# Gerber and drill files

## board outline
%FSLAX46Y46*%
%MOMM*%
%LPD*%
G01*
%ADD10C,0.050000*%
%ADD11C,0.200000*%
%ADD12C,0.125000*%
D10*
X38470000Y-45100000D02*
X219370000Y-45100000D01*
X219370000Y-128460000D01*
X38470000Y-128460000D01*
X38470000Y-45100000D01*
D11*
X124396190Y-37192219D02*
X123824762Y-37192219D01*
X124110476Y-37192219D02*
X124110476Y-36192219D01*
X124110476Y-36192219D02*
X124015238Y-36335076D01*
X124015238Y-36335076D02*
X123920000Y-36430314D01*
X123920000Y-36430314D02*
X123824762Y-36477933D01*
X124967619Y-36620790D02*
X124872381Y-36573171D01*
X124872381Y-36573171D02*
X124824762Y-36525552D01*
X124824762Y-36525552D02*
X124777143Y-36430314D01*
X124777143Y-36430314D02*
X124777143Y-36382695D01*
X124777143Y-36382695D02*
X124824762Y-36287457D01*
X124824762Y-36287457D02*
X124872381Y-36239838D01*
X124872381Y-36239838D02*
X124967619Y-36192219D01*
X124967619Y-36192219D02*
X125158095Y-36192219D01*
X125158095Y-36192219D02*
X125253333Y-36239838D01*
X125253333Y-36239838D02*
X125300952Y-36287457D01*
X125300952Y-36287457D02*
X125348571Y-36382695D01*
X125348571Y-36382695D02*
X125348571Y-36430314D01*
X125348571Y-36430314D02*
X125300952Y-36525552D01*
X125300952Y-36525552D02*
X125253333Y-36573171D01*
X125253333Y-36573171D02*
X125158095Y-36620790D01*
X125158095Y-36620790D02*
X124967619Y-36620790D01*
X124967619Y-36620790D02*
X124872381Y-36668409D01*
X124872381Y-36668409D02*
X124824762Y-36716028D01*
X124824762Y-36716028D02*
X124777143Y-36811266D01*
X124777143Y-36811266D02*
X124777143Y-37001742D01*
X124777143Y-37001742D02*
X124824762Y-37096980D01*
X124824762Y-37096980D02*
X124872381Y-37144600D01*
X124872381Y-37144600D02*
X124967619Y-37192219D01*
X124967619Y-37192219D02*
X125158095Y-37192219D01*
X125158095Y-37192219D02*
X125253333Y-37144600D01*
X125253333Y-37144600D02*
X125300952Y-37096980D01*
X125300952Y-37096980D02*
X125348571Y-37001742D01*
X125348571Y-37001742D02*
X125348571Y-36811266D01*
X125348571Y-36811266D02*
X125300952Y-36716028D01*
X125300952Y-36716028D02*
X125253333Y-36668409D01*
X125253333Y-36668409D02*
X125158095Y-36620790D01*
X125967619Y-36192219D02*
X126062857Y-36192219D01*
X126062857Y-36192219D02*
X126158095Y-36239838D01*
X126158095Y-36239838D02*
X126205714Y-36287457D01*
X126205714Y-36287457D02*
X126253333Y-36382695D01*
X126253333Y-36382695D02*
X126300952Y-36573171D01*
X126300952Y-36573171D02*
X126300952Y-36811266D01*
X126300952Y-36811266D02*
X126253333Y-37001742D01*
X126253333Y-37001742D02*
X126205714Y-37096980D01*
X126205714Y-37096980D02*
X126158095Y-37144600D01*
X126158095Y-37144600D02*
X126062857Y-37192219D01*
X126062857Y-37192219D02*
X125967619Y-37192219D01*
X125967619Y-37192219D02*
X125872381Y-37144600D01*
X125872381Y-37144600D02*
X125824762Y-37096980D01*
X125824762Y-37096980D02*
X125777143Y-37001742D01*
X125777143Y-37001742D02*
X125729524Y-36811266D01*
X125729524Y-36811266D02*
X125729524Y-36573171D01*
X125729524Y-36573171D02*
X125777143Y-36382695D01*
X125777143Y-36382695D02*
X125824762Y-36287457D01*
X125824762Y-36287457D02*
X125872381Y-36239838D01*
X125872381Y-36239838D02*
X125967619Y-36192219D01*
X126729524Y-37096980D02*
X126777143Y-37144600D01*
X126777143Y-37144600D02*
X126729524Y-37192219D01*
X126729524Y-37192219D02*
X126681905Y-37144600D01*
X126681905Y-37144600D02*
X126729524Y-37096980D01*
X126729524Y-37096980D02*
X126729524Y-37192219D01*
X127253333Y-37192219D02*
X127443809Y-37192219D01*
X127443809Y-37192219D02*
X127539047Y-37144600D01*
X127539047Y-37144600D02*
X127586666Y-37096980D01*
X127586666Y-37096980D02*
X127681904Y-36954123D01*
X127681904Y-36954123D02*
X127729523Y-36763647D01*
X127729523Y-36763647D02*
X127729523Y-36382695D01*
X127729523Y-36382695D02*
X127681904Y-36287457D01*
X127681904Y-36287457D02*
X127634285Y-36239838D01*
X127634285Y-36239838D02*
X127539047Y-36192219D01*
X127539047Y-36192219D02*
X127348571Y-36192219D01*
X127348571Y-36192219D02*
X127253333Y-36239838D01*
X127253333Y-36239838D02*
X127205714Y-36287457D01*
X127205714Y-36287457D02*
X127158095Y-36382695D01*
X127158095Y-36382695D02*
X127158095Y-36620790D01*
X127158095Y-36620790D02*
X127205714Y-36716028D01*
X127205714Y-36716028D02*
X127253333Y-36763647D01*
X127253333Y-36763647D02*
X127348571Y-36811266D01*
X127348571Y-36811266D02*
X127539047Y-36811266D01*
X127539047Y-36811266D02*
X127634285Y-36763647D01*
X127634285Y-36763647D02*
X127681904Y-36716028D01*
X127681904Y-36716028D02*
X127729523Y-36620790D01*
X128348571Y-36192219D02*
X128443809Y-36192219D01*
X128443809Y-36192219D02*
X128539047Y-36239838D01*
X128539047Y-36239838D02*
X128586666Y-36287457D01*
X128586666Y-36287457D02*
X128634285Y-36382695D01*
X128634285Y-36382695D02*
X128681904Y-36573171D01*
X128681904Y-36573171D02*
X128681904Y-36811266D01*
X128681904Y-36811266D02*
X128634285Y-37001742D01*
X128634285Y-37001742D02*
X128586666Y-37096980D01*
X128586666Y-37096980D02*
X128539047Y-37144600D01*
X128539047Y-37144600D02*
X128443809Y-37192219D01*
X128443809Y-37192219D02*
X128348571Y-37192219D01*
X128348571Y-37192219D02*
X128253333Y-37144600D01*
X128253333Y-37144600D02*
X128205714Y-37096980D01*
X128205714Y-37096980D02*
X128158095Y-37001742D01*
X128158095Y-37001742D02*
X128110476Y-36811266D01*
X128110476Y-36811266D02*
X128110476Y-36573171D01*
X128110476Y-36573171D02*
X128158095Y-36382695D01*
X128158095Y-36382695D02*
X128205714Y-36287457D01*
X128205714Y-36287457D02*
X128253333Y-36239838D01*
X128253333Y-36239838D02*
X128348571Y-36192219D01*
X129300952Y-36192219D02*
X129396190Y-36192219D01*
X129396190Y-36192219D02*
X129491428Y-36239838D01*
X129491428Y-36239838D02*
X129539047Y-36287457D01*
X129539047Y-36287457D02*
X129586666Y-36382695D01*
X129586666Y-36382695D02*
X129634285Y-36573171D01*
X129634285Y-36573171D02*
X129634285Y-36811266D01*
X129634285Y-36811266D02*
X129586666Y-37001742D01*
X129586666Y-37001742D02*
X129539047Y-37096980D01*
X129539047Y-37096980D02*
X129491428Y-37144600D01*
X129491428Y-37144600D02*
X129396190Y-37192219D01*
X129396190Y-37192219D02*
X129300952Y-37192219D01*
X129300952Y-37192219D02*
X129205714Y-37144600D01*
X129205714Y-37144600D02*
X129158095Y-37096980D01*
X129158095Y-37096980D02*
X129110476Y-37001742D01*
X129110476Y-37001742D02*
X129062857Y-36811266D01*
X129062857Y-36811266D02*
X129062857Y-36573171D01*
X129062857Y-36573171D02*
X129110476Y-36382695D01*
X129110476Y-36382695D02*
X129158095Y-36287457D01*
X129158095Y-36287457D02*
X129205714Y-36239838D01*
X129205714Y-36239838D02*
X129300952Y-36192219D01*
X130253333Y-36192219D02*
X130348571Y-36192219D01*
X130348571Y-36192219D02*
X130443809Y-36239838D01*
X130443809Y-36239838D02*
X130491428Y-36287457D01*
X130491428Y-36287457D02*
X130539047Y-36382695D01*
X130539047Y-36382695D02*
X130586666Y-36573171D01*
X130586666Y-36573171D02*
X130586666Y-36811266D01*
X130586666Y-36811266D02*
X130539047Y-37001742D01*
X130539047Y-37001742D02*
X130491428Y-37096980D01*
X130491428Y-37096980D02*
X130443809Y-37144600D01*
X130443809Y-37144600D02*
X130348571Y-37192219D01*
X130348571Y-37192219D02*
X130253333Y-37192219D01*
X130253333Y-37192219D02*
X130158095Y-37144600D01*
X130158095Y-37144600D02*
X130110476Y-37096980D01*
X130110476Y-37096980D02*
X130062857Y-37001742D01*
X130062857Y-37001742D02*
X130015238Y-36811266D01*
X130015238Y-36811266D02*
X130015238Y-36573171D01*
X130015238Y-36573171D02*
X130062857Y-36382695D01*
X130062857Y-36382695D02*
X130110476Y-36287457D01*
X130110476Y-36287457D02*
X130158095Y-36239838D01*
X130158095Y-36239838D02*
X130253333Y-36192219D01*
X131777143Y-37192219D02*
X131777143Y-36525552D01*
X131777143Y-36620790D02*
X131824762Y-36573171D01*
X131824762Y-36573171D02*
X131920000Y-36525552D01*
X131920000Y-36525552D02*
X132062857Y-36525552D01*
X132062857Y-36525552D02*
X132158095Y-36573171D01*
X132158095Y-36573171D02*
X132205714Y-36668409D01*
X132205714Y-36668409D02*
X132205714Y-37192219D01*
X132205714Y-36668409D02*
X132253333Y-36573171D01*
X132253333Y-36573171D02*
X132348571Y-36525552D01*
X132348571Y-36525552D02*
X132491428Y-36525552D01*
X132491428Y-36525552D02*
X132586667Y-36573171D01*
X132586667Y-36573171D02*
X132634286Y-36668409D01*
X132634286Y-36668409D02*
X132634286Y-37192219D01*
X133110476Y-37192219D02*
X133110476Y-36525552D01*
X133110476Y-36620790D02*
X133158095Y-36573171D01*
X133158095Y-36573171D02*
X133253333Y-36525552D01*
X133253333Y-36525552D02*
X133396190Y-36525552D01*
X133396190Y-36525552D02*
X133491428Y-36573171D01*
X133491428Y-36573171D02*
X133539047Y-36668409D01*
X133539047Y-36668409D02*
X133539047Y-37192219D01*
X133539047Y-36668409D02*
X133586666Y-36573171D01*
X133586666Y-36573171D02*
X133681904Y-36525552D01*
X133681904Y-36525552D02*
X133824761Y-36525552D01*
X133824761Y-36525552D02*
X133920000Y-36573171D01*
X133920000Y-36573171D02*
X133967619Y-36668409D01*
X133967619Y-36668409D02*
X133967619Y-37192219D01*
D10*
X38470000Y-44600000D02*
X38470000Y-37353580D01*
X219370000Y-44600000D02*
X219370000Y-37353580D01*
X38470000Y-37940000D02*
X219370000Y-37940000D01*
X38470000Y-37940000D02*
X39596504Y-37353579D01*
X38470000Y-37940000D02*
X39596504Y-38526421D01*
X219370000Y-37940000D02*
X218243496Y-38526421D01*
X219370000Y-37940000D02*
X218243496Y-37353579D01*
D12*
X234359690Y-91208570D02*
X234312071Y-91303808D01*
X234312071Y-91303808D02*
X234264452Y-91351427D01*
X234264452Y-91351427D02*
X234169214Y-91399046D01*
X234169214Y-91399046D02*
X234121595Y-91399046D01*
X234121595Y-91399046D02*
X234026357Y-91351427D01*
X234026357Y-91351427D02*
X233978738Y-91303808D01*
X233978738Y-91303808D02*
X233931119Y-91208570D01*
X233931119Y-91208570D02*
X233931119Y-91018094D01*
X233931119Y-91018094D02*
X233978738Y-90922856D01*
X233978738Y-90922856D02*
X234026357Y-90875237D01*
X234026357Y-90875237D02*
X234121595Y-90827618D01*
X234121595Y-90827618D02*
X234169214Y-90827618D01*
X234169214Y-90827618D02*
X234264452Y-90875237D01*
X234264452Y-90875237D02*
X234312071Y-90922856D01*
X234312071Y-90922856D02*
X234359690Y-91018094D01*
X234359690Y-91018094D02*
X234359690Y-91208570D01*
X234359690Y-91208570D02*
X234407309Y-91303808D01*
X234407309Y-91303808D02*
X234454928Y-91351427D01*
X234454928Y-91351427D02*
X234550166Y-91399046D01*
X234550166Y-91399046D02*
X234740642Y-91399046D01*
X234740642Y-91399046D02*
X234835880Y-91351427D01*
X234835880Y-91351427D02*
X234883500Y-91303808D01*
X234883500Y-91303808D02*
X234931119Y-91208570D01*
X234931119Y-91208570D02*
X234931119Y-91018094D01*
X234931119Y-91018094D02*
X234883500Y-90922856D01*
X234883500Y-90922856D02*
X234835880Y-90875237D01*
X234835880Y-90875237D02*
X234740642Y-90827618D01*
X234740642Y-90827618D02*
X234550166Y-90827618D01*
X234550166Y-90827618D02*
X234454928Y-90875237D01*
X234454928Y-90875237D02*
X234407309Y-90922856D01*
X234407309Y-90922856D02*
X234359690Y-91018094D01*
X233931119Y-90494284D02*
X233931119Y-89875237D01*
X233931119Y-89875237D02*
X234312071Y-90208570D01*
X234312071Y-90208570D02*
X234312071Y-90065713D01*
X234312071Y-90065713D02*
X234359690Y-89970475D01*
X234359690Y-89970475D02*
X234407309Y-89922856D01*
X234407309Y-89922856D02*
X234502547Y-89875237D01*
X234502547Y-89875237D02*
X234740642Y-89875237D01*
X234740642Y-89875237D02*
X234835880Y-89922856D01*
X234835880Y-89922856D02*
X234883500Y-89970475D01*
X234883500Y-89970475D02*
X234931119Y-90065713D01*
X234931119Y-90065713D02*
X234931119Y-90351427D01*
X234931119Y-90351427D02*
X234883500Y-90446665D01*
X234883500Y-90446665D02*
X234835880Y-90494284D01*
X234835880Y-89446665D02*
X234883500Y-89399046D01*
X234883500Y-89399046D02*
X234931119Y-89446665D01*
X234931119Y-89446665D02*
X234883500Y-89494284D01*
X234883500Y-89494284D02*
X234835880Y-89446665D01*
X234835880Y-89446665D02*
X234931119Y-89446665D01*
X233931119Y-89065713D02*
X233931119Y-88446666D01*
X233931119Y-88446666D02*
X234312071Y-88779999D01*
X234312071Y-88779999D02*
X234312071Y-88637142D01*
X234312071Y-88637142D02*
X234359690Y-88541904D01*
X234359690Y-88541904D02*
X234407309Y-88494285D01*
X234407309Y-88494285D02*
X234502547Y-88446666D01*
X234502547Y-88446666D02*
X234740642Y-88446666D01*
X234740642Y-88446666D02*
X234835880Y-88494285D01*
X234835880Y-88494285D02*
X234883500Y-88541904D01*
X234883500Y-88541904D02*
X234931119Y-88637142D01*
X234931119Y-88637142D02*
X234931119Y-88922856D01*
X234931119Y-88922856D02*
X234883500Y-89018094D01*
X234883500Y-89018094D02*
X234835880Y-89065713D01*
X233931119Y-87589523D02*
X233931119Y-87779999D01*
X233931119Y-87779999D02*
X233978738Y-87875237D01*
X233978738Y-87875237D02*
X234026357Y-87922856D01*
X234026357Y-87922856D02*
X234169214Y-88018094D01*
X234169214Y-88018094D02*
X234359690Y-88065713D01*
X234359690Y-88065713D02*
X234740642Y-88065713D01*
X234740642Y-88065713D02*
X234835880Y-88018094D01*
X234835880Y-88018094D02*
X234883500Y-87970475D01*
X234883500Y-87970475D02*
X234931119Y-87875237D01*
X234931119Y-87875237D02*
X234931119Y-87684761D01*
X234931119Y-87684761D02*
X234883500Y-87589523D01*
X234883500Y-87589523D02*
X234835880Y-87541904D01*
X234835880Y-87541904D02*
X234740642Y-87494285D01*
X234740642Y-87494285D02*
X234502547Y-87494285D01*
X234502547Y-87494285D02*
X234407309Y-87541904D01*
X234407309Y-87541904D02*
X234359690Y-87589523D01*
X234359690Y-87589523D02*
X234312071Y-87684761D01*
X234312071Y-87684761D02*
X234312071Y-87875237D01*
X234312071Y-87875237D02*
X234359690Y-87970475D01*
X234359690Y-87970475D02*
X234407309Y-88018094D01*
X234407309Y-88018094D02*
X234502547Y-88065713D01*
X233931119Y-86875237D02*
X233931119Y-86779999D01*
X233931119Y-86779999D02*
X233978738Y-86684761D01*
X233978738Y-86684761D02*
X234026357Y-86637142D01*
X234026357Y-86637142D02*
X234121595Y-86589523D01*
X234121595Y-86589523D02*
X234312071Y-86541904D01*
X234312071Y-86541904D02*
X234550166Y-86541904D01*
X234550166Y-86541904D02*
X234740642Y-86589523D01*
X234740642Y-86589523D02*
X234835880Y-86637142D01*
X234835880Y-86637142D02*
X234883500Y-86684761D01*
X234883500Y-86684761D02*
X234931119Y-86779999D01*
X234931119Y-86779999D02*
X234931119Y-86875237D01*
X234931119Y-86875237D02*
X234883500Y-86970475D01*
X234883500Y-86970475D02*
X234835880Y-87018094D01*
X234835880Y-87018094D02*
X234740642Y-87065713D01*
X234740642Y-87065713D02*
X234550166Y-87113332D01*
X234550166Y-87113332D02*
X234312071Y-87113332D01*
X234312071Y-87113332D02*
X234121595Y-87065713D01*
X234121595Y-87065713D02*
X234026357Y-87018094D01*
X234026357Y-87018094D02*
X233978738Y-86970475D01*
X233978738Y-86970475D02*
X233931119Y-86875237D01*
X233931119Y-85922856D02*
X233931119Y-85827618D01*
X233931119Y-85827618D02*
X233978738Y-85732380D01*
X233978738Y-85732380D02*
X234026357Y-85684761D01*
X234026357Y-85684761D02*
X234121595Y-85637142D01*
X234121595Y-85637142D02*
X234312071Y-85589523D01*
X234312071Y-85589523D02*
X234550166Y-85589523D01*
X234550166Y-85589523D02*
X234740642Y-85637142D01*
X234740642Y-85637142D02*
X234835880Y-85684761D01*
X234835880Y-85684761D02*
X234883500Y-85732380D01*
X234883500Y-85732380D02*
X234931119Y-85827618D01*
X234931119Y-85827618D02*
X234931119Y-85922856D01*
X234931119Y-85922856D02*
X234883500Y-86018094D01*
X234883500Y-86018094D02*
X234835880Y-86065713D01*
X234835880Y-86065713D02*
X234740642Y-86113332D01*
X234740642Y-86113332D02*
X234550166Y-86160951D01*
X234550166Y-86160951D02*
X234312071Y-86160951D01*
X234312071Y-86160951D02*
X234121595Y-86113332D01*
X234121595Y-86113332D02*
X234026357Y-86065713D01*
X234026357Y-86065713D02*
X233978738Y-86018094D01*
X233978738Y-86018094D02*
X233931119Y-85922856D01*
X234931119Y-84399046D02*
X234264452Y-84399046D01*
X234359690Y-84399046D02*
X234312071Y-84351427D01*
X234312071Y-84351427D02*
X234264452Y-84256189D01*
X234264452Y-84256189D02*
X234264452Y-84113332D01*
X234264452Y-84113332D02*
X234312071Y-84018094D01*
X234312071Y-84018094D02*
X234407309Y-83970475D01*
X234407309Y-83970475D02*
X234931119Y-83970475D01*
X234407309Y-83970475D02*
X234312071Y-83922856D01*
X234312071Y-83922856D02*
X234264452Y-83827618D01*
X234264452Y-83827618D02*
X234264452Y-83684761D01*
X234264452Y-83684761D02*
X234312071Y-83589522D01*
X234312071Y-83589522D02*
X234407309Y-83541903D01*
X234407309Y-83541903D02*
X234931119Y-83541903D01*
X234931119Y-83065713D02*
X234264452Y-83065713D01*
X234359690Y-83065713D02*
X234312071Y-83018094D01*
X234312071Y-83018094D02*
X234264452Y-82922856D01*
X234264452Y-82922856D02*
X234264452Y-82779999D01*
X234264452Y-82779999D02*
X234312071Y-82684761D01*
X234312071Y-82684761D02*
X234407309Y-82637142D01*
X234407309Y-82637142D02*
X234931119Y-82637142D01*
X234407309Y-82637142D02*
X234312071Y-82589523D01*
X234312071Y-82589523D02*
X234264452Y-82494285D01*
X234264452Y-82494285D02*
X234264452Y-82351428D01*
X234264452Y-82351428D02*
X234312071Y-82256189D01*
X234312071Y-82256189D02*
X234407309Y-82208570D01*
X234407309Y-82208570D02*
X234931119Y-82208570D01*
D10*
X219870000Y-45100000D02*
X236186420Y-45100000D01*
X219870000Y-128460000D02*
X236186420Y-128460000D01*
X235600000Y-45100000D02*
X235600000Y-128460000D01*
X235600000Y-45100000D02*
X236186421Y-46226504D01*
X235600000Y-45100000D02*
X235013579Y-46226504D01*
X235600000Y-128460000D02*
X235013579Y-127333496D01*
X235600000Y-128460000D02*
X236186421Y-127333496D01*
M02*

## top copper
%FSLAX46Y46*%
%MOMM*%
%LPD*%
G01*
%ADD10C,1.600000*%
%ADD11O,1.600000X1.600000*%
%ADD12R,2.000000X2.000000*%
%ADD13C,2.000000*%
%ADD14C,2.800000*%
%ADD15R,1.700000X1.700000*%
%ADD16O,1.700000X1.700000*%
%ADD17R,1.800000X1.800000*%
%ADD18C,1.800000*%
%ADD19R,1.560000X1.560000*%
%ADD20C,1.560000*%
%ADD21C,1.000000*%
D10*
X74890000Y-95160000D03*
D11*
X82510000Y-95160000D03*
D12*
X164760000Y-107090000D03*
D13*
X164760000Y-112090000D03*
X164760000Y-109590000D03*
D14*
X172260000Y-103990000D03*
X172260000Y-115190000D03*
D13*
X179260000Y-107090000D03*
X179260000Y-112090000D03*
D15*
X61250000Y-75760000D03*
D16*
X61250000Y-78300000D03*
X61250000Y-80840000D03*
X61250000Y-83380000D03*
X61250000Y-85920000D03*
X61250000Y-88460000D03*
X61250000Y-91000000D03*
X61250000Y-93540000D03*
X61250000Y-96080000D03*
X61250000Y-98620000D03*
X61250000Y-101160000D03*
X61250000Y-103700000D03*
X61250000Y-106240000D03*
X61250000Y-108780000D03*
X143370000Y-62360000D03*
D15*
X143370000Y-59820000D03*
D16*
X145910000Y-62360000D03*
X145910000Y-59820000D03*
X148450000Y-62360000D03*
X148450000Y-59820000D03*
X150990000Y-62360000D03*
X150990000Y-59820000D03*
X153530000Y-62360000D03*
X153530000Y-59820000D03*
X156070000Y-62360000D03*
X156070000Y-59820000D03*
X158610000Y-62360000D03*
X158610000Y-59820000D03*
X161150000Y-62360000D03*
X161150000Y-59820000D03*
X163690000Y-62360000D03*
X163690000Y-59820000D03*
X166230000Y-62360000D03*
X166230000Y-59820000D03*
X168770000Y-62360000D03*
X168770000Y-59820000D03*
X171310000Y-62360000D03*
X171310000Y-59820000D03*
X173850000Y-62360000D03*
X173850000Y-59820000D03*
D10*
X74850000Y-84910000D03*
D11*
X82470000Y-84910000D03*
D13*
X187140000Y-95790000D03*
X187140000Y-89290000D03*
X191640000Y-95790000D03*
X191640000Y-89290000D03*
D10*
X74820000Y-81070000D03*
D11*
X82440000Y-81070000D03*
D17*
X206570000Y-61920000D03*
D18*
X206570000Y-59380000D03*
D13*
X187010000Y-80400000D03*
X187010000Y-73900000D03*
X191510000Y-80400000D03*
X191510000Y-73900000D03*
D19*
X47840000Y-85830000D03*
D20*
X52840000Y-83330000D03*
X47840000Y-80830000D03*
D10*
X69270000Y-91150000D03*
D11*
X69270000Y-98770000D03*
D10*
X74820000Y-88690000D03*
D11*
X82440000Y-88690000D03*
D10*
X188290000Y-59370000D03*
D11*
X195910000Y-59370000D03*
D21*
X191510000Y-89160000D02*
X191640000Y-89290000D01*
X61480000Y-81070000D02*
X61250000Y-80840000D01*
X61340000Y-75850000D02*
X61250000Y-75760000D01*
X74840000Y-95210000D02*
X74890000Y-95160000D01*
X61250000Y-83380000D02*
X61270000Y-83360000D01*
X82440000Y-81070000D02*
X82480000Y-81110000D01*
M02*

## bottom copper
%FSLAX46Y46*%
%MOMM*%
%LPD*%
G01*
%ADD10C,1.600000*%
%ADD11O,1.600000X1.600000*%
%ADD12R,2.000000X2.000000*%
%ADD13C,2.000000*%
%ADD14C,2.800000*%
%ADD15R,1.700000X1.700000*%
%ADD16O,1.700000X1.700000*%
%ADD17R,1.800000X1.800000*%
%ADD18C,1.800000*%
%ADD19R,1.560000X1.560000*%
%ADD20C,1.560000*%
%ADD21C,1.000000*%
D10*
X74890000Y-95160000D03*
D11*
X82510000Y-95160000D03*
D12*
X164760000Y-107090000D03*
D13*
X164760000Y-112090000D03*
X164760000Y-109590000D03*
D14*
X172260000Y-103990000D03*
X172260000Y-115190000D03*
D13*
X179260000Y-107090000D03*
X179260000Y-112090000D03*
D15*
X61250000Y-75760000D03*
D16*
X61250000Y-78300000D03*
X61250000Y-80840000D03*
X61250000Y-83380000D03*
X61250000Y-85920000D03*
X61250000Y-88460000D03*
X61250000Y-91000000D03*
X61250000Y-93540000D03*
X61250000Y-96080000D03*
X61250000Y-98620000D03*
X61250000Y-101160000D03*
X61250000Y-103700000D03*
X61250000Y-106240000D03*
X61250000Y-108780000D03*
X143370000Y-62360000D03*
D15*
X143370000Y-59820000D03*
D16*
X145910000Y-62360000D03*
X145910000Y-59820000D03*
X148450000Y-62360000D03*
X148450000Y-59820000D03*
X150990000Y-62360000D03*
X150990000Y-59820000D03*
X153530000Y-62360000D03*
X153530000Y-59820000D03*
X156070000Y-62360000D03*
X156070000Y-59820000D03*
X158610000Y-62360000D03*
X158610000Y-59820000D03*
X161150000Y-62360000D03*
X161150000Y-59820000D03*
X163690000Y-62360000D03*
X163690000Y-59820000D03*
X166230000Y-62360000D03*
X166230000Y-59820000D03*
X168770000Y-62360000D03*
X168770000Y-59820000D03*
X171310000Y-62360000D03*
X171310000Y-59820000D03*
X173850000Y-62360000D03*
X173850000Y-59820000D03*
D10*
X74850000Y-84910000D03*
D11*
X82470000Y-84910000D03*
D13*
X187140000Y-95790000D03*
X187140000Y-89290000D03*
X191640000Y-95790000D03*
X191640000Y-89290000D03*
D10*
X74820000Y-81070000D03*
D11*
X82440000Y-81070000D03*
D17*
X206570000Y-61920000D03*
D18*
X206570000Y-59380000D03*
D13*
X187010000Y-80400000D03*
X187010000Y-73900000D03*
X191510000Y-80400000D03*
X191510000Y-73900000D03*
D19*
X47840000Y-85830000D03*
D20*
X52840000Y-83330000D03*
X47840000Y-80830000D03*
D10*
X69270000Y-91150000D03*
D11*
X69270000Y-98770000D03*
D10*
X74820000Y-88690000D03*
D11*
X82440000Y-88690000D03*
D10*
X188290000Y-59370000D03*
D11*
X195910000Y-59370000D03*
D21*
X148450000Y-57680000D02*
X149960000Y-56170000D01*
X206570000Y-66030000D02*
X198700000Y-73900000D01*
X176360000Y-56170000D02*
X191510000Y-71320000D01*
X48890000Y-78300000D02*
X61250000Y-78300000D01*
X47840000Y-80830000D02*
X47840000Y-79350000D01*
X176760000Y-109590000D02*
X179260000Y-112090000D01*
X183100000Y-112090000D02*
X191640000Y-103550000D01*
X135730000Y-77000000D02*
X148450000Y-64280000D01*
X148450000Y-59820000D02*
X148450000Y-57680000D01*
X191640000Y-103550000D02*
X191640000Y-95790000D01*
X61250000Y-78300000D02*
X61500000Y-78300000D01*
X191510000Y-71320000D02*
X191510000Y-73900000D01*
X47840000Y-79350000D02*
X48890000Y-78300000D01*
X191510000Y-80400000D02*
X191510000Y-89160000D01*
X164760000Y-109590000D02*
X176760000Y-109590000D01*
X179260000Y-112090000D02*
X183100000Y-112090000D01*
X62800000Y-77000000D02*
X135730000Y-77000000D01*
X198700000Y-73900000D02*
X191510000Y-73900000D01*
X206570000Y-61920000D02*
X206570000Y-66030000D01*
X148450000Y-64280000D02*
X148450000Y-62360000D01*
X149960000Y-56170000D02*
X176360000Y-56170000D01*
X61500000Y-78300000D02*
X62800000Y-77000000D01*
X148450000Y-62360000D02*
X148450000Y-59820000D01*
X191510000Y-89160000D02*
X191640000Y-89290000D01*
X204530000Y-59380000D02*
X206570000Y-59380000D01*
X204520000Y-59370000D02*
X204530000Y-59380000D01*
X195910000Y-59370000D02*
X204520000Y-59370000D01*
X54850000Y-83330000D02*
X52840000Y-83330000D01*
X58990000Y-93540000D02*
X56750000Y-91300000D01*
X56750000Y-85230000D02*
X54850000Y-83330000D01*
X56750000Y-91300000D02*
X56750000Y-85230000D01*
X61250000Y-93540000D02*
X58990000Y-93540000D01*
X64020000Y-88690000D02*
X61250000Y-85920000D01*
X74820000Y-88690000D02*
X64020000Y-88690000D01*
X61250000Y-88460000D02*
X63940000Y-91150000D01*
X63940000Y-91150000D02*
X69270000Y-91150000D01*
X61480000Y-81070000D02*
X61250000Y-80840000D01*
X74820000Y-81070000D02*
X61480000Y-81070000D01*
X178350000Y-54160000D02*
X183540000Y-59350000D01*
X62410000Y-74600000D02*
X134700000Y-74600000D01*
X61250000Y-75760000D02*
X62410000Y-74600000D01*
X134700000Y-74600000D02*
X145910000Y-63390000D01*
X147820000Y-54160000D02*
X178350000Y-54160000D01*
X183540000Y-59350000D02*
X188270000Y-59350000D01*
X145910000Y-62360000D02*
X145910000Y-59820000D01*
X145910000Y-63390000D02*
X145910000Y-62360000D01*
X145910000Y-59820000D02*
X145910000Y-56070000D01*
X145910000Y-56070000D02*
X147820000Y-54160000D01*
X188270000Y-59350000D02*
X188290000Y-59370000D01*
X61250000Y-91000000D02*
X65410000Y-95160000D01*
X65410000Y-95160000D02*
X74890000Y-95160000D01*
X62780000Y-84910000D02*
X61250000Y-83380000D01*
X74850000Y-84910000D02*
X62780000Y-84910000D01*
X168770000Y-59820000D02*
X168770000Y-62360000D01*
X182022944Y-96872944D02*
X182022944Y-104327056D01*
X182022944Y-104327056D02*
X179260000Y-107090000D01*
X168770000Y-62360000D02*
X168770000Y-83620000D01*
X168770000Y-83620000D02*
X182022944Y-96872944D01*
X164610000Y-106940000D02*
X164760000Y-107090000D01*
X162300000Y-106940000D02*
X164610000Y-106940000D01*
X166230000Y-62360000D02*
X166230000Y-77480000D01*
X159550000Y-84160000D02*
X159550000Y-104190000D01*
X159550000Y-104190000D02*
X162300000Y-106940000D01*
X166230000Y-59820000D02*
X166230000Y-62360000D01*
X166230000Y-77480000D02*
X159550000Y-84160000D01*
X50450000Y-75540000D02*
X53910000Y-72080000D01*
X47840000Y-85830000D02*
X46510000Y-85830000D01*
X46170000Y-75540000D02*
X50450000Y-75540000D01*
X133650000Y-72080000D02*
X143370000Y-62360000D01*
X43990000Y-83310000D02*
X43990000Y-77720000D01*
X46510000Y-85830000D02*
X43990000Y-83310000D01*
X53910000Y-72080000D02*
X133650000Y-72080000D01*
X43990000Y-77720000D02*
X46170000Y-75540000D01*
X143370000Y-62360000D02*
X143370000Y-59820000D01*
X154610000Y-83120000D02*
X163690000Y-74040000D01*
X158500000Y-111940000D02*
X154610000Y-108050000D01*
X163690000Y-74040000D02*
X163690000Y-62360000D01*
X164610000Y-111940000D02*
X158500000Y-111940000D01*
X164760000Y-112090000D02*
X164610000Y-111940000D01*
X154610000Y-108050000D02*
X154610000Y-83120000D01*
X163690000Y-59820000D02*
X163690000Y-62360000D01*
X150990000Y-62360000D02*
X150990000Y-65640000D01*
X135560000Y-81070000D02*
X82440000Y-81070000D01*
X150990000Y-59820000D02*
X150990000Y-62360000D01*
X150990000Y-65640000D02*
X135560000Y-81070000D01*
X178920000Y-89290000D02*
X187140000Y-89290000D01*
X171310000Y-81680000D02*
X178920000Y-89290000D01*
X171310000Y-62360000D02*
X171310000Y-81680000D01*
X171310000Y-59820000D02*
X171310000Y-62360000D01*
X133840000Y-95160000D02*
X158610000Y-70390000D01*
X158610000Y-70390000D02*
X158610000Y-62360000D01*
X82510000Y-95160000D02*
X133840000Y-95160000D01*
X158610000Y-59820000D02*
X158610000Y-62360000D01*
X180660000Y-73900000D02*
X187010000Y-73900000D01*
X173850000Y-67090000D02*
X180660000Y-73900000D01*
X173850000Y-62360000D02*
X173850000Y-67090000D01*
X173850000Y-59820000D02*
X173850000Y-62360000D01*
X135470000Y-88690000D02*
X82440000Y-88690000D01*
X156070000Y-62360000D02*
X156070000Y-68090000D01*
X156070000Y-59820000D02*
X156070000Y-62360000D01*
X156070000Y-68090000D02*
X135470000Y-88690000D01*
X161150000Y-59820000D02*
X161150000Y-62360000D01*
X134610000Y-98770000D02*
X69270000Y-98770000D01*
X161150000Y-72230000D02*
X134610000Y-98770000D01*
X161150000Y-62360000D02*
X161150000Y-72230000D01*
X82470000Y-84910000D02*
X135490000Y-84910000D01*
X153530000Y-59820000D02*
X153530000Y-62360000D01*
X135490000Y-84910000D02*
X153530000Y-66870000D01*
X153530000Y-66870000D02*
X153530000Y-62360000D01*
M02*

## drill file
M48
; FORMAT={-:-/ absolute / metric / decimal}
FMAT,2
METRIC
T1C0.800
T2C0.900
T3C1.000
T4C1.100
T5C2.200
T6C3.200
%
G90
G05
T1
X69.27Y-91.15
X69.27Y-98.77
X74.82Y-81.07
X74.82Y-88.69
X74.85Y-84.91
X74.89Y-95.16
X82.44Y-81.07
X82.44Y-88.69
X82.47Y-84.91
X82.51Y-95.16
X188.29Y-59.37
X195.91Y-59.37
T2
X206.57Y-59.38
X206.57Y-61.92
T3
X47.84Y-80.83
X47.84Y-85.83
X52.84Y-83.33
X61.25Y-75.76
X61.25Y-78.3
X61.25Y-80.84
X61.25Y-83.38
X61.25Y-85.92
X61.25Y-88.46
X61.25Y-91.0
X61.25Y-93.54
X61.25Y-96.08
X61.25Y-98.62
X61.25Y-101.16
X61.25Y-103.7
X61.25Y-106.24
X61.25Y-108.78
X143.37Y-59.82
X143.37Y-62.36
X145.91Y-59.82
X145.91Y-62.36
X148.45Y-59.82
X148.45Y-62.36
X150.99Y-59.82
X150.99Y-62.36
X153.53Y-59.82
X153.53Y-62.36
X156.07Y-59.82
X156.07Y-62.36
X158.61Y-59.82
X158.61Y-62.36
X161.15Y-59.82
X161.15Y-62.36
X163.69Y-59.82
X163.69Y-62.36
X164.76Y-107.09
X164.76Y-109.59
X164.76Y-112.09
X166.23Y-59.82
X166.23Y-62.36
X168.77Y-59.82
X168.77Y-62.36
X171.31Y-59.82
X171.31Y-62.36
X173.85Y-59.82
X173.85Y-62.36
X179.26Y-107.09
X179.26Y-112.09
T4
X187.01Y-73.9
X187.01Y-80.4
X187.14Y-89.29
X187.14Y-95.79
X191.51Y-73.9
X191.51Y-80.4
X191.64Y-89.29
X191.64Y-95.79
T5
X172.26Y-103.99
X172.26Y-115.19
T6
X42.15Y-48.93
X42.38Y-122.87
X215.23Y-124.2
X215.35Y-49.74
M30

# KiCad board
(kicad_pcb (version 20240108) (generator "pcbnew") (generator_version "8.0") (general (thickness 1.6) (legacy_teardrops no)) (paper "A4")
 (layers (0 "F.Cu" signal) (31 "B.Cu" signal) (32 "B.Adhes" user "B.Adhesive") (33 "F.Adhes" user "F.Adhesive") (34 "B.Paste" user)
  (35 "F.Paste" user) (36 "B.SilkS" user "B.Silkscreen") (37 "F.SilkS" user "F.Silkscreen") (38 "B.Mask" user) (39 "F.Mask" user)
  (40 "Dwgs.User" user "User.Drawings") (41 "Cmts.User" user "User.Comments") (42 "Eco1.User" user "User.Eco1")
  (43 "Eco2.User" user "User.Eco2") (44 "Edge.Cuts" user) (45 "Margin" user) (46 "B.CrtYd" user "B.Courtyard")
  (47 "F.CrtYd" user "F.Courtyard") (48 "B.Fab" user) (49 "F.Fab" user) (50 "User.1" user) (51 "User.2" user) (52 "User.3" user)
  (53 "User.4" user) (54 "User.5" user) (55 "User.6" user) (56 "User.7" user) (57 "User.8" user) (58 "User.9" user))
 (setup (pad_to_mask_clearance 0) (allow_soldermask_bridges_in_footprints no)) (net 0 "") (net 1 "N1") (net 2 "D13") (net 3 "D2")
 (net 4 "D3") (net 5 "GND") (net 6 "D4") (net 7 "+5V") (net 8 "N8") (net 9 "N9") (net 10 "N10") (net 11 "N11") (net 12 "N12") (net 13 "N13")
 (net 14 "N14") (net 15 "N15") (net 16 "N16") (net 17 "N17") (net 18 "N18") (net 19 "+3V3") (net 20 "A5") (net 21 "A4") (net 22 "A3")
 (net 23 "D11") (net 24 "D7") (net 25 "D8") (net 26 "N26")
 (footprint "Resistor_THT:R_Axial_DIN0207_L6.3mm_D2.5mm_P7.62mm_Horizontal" (layer "F.Cu") (at 74.89 95.16)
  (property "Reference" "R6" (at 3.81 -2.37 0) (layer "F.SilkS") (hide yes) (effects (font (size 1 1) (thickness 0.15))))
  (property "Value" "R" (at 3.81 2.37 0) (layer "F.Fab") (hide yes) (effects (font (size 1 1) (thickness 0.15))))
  (pad "1" thru_hole circle (at 0 0) (size 1.6 1.6) (drill 0.8) (layers "*.Cu" "*.Mask") (remove_unused_layers no) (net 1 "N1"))
  (pad "2" thru_hole oval (at 7.62 0) (size 1.6 1.6) (drill 0.8) (layers "*.Cu" "*.Mask") (remove_unused_layers no) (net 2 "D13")))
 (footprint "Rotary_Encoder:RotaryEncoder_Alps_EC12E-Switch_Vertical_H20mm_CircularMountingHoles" (layer "F.Cu") (at 164.76 107.09)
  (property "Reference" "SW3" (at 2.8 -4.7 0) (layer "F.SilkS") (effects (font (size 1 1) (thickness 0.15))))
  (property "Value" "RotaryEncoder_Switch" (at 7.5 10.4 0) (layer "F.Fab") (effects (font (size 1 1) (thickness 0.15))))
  (pad "A" thru_hole rect (at 0 0) (size 2 2) (drill 1) (layers "*.Cu" "*.Mask") (remove_unused_layers no) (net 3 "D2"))
  (pad "B" thru_hole circle (at 0 5) (size 2 2) (drill 1) (layers "*.Cu" "*.Mask") (remove_unused_layers no) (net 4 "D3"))
  (pad "C" thru_hole circle (at 0 2.5) (size 2 2) (drill 1) (layers "*.Cu" "*.Mask") (remove_unused_layers no) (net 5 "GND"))
  (pad "MP" thru_hole circle (at 7.5 -3.1) (size 2.8 2.8) (drill 2.2) (layers "*.Cu" "*.Mask") (remove_unused_layers no))
  (pad "MP" thru_hole circle (at 7.5 8.1) (size 2.8 2.8) (drill 2.2) (layers "*.Cu" "*.Mask") (remove_unused_layers no))
  (pad "S1" thru_hole circle (at 14.5 0) (size 2 2) (drill 1) (layers "*.Cu" "*.Mask") (remove_unused_layers no) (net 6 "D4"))
  (pad "S2" thru_hole circle (at 14.5 5) (size 2 2) (drill 1) (layers "*.Cu" "*.Mask") (remove_unused_layers no) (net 5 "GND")))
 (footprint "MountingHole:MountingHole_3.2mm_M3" (layer "F.Cu") (at 215.23 124.2)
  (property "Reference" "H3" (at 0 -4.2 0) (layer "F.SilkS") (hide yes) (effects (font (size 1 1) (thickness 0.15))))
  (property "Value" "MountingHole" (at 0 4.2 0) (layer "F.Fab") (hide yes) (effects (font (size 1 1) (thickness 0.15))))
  (pad "" np_thru_hole circle (at 0 0) (size 3.2 3.2) (drill 3.2) (layers "*.Cu" "*.Mask")))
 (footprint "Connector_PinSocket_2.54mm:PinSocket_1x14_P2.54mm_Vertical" (layer "F.Cu") (at 61.25 75.76)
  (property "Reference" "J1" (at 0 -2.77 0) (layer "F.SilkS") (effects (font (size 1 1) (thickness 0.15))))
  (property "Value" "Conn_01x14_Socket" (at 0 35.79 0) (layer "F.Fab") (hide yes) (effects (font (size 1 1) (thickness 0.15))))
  (pad "1" thru_hole rect (at 0 0) (size 1.7 1.7) (drill 1) (layers "*.Cu" "*.Mask") (remove_unused_layers no) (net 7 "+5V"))
  (pad "2" thru_hole oval (at 0 2.54) (size 1.7 1.7) (drill 1) (layers "*.Cu" "*.Mask") (remove_unused_layers no) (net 5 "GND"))
  (pad "3" thru_hole oval (at 0 5.08) (size 1.7 1.7) (drill 1) (layers "*.Cu" "*.Mask") (remove_unused_layers no) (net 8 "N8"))
  (pad "4" thru_hole oval (at 0 7.62) (size 1.7 1.7) (drill 1) (layers "*.Cu" "*.Mask") (remove_unused_layers no) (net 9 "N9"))
  (pad "5" thru_hole oval (at 0 10.16) (size 1.7 1.7) (drill 1) (layers "*.Cu" "*.Mask") (remove_unused_layers no) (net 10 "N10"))
  (pad "6" thru_hole oval (at 0 12.7) (size 1.7 1.7) (drill 1) (layers "*.Cu" "*.Mask") (remove_unused_layers no) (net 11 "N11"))
  (pad "7" thru_hole oval (at 0 15.24) (size 1.7 1.7) (drill 1) (layers "*.Cu" "*.Mask") (remove_unused_layers no) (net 1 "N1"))
  (pad "8" thru_hole oval (at 0 17.78) (size 1.7 1.7) (drill 1) (layers "*.Cu" "*.Mask") (remove_unused_layers no) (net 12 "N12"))
  (pad "9" thru_hole oval (at 0 20.32) (size 1.7 1.7) (drill 1) (layers "*.Cu" "*.Mask") (remove_unused_layers no) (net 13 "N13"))
  (pad "10" thru_hole oval (at 0 22.86) (size 1.7 1.7) (drill 1) (layers "*.Cu" "*.Mask") (remove_unused_layers no) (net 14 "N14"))
  (pad "11" thru_hole oval (at 0 25.4) (size 1.7 1.7) (drill 1) (layers "*.Cu" "*.Mask") (remove_unused_layers no) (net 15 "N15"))
  (pad "12" thru_hole oval (at 0 27.94) (size 1.7 1.7) (drill 1) (layers "*.Cu" "*.Mask") (remove_unused_layers no) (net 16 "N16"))
  (pad "13" thru_hole oval (at 0 30.48) (size 1.7 1.7) (drill 1) (layers "*.Cu" "*.Mask") (remove_unused_layers no) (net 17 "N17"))
  (pad "14" thru_hole oval (at 0 33.02) (size 1.7 1.7) (drill 1) (layers "*.Cu" "*.Mask") (remove_unused_layers no) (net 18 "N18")))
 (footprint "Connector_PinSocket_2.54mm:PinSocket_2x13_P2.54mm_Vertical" (layer "F.Cu") (at 143.37 59.82 90)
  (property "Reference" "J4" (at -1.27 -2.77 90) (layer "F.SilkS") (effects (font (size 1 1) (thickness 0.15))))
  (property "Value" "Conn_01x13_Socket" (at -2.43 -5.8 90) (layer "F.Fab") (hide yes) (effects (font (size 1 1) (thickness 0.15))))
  (pad "1" thru_hole oval (at -2.54 0 90) (size 1.7 1.7) (drill 1) (layers "*.Cu" "*.Mask") (remove_unused_layers no) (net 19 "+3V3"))
  (pad "1" thru_hole rect (at 0 0 90) (size 1.7 1.7) (drill 1) (layers "*.Cu" "*.Mask") (remove_unused_layers no) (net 19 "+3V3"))
  (pad "2" thru_hole oval (at -2.54 2.54 90) (size 1.7 1.7) (drill 1) (layers "*.Cu" "*.Mask") (remove_unused_layers no) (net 7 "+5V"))
  (pad "2" thru_hole oval (at 0 2.54 90) (size 1.7 1.7) (drill 1) (layers "*.Cu" "*.Mask") (remove_unused_layers no) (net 7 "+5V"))
  (pad "3" thru_hole oval (at -2.54 5.08 90) (size 1.7 1.7) (drill 1) (layers "*.Cu" "*.Mask") (remove_unused_layers no) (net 5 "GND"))
  (pad "3" thru_hole oval (at 0 5.08 90) (size 1.7 1.7) (drill 1) (layers "*.Cu" "*.Mask") (remove_unused_layers no) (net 5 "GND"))
  (pad "4" thru_hole oval (at -2.54 7.62 90) (size 1.7 1.7) (drill 1) (layers "*.Cu" "*.Mask") (remove_unused_layers no) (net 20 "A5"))
  (pad "4" thru_hole oval (at 0 7.62 90) (size 1.7 1.7) (drill 1) (layers "*.Cu" "*.Mask") (remove_unused_layers no) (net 20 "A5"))
  (pad "5" thru_hole oval (at -2.54 10.16 90) (size 1.7 1.7) (drill 1) (layers "*.Cu" "*.Mask") (remove_unused_layers no) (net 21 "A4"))
  (pad "5" thru_hole oval (at 0 10.16 90) (size 1.7 1.7) (drill 1) (layers "*.Cu" "*.Mask") (remove_unused_layers no) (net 21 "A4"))
  (pad "6" thru_hole oval (at -2.54 12.7 90) (size 1.7 1.7) (drill 1) (layers "*.Cu" "*.Mask") (remove_unused_layers no) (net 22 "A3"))
  (pad "6" thru_hole oval (at 0 12.7 90) (size 1.7 1.7) (drill 1) (layers "*.Cu" "*.Mask") (remove_unused_layers no) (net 22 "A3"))
  (pad "7" thru_hole oval (at -2.54 15.24 90) (size 1.7 1.7) (drill 1) (layers "*.Cu" "*.Mask") (remove_unused_layers no) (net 2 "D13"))
  (pad "7" thru_hole oval (at 0 15.24 90) (size 1.7 1.7) (drill 1) (layers "*.Cu" "*.Mask") (remove_unused_layers no) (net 2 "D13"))
  (pad "8" thru_hole oval (at -2.54 17.78 90) (size 1.7 1.7) (drill 1) (layers "*.Cu" "*.Mask") (remove_unused_layers no) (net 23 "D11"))
  (pad "8" thru_hole oval (at 0 17.78 90) (size 1.7 1.7) (drill 1) (layers "*.Cu" "*.Mask") (remove_unused_layers no) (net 23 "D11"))
  (pad "9" thru_hole oval (at -2.54 20.32 90) (size 1.7 1.7) (drill 1) (layers "*.Cu" "*.Mask") (remove_unused_layers no) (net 4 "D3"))
  (pad "9" thru_hole oval (at 0 20.32 90) (size 1.7 1.7) (drill 1) (layers "*.Cu" "*.Mask") (remove_unused_layers no) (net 4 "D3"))
  (pad "10" thru_hole oval (at -2.54 22.86 90) (size 1.7 1.7) (drill 1) (layers "*.Cu" "*.Mask") (remove_unused_layers no) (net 3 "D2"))
  (pad "10" thru_hole oval (at 0 22.86 90) (size 1.7 1.7) (drill 1) (layers "*.Cu" "*.Mask") (remove_unused_layers no) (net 3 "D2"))
  (pad "11" thru_hole oval (at -2.54 25.4 90) (size 1.7 1.7) (drill 1) (layers "*.Cu" "*.Mask") (remove_unused_layers no) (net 6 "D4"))
  (pad "11" thru_hole oval (at 0 25.4 90) (size 1.7 1.7) (drill 1) (layers "*.Cu" "*.Mask") (remove_unused_layers no) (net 6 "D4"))
  (pad "12" thru_hole oval (at -2.54 27.94 90) (size 1.7 1.7) (drill 1) (layers "*.Cu" "*.Mask") (remove_unused_layers no) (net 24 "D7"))
  (pad "12" thru_hole oval (at 0 27.94 90) (size 1.7 1.7) (drill 1) (layers "*.Cu" "*.Mask") (remove_unused_layers no) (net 24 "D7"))
  (pad "13" thru_hole oval (at -2.54 30.48 90) (size 1.7 1.7) (drill 1) (layers "*.Cu" "*.Mask") (remove_unused_layers no) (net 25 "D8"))
  (pad "13" thru_hole oval (at 0 30.48 90) (size 1.7 1.7) (drill 1) (layers "*.Cu" "*.Mask") (remove_unused_layers no) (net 25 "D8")))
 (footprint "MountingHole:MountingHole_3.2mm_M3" (layer "F.Cu") (at 42.15 48.93)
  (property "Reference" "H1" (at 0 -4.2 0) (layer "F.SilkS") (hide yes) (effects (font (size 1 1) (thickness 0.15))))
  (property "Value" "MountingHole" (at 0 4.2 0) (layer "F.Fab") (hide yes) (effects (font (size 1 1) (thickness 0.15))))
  (pad "" np_thru_hole circle (at 0 0) (size 3.2 3.2) (drill 3.2) (layers "*.Cu" "*.Mask")))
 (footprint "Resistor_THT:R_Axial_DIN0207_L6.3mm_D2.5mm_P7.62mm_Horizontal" (layer "F.Cu") (at 74.85 84.91)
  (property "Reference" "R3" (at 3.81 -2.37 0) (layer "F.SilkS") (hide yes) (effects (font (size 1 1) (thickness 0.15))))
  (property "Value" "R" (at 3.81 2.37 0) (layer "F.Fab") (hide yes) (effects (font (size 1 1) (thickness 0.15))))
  (pad "1" thru_hole circle (at 0 0) (size 1.6 1.6) (drill 0.8) (layers "*.Cu" "*.Mask") (remove_unused_layers no) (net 9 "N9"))
  (pad "2" thru_hole oval (at 7.62 0) (size 1.6 1.6) (drill 0.8) (layers "*.Cu" "*.Mask") (remove_unused_layers no) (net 21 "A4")))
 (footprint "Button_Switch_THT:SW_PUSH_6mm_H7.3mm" (layer "F.Cu") (at 187.14 95.79 90)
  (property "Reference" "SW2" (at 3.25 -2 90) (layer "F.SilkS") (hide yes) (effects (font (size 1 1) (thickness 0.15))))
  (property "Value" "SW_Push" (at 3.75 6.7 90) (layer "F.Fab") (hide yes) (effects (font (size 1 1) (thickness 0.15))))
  (pad "1" thru_hole circle (at 0 0 180) (size 2 2) (drill 1.1) (layers "*.Cu" "*.Mask") (remove_unused_layers no) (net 24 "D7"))
  (pad "1" thru_hole circle (at 6.5 0 180) (size 2 2) (drill 1.1) (layers "*.Cu" "*.Mask") (remove_unused_layers no) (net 24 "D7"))
  (pad "2" thru_hole circle (at 0 4.5 180) (size 2 2) (drill 1.1) (layers "*.Cu" "*.Mask") (remove_unused_layers no) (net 5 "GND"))
  (pad "2" thru_hole circle (at 6.5 4.5 180) (size 2 2) (drill 1.1) (layers "*.Cu" "*.Mask") (remove_unused_layers no) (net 5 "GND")))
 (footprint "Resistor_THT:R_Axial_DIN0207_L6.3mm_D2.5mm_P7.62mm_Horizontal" (layer "F.Cu") (at 74.82 81.07)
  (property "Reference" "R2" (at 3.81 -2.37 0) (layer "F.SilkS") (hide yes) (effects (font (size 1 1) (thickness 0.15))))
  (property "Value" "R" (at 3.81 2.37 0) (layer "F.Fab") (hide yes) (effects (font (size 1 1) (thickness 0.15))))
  (pad "1" thru_hole circle (at 0 0) (size 1.6 1.6) (drill 0.8) (layers "*.Cu" "*.Mask") (remove_unused_layers no) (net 8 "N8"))
  (pad "2" thru_hole oval (at 7.62 0) (size 1.6 1.6) (drill 0.8) (layers "*.Cu" "*.Mask") (remove_unused_layers no) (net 20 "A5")))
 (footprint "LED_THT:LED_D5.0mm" (layer "F.Cu") (at 206.57 61.92 90)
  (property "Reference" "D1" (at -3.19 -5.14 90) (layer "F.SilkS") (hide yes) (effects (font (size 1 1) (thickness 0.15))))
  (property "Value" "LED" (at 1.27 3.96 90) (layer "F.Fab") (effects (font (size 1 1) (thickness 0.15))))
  (pad "1" thru_hole rect (at 0 0 90) (size 1.8 1.8) (drill 0.9) (layers "*.Cu" "*.Mask") (remove_unused_layers no) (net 5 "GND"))
  (pad "2" thru_hole circle (at 2.54 0 90) (size 1.8 1.8) (drill 0.9) (layers "*.Cu" "*.Mask") (remove_unused_layers no) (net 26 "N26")))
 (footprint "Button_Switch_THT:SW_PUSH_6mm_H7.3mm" (layer "F.Cu") (at 187.01 80.4 90)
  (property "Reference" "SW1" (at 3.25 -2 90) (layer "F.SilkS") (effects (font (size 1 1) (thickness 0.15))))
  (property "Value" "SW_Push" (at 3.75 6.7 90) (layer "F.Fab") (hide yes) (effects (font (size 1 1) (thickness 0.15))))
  (pad "1" thru_hole circle (at 0 0 180) (size 2 2) (drill 1.1) (layers "*.Cu" "*.Mask") (remove_unused_layers no) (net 25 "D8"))
  (pad "1" thru_hole circle (at 6.5 0 180) (size 2 2) (drill 1.1) (layers "*.Cu" "*.Mask") (remove_unused_layers no) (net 25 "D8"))
  (pad "2" thru_hole circle (at 0 4.5 180) (size 2 2) (drill 1.1) (layers "*.Cu" "*.Mask") (remove_unused_layers no) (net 5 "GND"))
  (pad "2" thru_hole circle (at 6.5 4.5 180) (size 2 2) (drill 1.1) (layers "*.Cu" "*.Mask") (remove_unused_layers no) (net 5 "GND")))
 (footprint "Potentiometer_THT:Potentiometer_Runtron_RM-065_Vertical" (layer "F.Cu") (at 47.84 85.83 90)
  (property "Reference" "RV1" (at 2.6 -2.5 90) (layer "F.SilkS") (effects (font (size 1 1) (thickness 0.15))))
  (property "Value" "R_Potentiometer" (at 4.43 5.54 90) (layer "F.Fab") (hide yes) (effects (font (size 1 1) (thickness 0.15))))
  (pad "1" thru_hole rect (at 0 0 90) (size 1.56 1.56) (drill 1) (layers "*.Cu" "*.Mask") (remove_unused_layers no) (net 19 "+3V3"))
  (pad "2" thru_hole circle (at 2.5 5 90) (size 1.56 1.56) (drill 1) (layers "*.Cu" "*.Mask") (remove_unused_layers no) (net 12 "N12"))
  (pad "3" thru_hole circle (at 5 0 90) (size 1.56 1.56) (drill 1) (layers "*.Cu" "*.Mask") (remove_unused_layers no) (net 5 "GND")))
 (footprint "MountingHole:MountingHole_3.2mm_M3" (layer "F.Cu") (at 42.38 122.87)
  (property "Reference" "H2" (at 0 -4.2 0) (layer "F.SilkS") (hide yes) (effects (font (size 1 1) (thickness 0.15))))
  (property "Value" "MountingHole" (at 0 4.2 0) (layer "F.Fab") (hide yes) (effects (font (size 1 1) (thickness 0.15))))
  (pad "" np_thru_hole circle (at 0 0) (size 3.2 3.2) (drill 3.2) (layers "*.Cu" "*.Mask")))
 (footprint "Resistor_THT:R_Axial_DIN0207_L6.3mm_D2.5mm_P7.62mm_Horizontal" (layer "F.Cu") (at 69.27 91.15 -90)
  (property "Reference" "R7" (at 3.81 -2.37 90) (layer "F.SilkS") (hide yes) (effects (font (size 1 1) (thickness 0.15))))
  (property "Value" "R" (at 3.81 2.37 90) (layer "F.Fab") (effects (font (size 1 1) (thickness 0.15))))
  (pad "1" thru_hole circle (at 0 0 270) (size 1.6 1.6) (drill 0.8) (layers "*.Cu" "*.Mask") (remove_unused_layers no) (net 11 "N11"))
  (pad "2" thru_hole oval (at 7.62 0 270) (size 1.6 1.6) (drill 0.8) (layers "*.Cu" "*.Mask") (remove_unused_layers no) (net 23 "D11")))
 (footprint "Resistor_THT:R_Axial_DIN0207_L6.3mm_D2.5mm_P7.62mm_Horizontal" (layer "F.Cu") (at 74.82 88.69)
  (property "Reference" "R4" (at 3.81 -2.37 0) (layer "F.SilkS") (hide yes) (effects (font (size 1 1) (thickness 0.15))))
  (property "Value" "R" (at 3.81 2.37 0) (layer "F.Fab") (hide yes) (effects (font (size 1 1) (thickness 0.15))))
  (pad "1" thru_hole circle (at 0 0) (size 1.6 1.6) (drill 0.8) (layers "*.Cu" "*.Mask") (remove_unused_layers no) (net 10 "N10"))
  (pad "2" thru_hole oval (at 7.62 0) (size 1.6 1.6) (drill 0.8) (layers "*.Cu" "*.Mask") (remove_unused_layers no) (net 22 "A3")))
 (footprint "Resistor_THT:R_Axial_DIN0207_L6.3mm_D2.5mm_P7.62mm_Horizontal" (layer "F.Cu") (at 188.29 59.37)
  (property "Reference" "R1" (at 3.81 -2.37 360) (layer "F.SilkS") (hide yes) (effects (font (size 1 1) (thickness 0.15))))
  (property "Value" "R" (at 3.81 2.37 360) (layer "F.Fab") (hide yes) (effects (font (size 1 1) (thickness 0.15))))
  (pad "1" thru_hole circle (at 0 0) (size 1.6 1.6) (drill 0.8) (layers "*.Cu" "*.Mask") (remove_unused_layers no) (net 7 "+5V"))
  (pad "2" thru_hole oval (at 7.62 0) (size 1.6 1.6) (drill 0.8) (layers "*.Cu" "*.Mask") (remove_unused_layers no) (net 26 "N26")))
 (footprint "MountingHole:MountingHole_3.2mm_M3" (layer "F.Cu") (at 215.35 49.74)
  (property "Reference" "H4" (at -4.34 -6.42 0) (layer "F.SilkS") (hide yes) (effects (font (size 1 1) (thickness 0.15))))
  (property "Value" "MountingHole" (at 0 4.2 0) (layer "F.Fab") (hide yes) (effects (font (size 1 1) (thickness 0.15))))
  (pad "" np_thru_hole circle (at 0 0) (size 3.2 3.2) (drill 3.2) (layers "*.Cu" "*.Mask")))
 (gr_rect (start 38.47 45.1) (end 219.37 128.46) (stroke (width 0.05) (type default)) (fill none) (layer "Edge.Cuts"))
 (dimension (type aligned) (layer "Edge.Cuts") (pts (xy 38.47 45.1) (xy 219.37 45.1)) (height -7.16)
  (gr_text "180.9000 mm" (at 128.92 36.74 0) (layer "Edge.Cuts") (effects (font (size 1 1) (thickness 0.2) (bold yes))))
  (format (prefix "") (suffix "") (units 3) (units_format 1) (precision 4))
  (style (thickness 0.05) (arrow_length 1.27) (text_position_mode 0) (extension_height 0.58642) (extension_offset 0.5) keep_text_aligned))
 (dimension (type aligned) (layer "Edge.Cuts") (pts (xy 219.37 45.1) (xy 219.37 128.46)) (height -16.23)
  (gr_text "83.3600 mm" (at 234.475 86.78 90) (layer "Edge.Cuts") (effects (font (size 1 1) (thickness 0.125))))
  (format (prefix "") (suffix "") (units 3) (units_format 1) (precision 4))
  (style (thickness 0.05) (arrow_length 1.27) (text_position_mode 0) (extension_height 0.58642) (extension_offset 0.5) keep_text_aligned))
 (segment (start 191.51 89.16) (end 191.64 89.29) (width 1) (layer "F.Cu") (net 5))
 (segment (start 148.45 57.68) (end 149.96 56.17) (width 1) (layer "B.Cu") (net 5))
 (segment (start 206.57 66.03) (end 198.7 73.9) (width 1) (layer "B.Cu") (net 5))
 (segment (start 176.36 56.17) (end 191.51 71.32) (width 1) (layer "B.Cu") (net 5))
 (segment (start 48.89 78.3) (end 61.25 78.3) (width 1) (layer "B.Cu") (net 5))
 (segment (start 47.84 80.83) (end 47.84 79.35) (width 1) (layer "B.Cu") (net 5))
 (segment (start 176.76 109.59) (end 179.26 112.09) (width 1) (layer "B.Cu") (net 5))
 (segment (start 183.1 112.09) (end 191.64 103.55) (width 1) (layer "B.Cu") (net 5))
 (segment (start 135.73 77) (end 148.45 64.28) (width 1) (layer "B.Cu") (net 5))
 (segment (start 148.45 59.82) (end 148.45 57.68) (width 1) (layer "B.Cu") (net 5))
 (segment (start 191.64 103.55) (end 191.64 95.79) (width 1) (layer "B.Cu") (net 5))
 (segment (start 61.25 78.3) (end 61.5 78.3) (width 1) (layer "B.Cu") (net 5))
 (segment (start 191.51 71.32) (end 191.51 73.9) (width 1) (layer "B.Cu") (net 5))
 (segment (start 47.84 79.35) (end 48.89 78.3) (width 1) (layer "B.Cu") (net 5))
 (segment (start 191.51 80.4) (end 191.51 89.16) (width 1) (layer "B.Cu") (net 5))
 (segment (start 164.76 109.59) (end 176.76 109.59) (width 1) (layer "B.Cu") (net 5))
 (segment (start 179.26 112.09) (end 183.1 112.09) (width 1) (layer "B.Cu") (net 5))
 (segment (start 62.8 77) (end 135.73 77) (width 1) (layer "B.Cu") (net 5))
 (segment (start 198.7 73.9) (end 191.51 73.9) (width 1) (layer "B.Cu") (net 5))
 (segment (start 206.57 61.92) (end 206.57 66.03) (width 1) (layer "B.Cu") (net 5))
 (segment (start 148.45 64.28) (end 148.45 62.36) (width 1) (layer "B.Cu") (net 5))
 (segment (start 149.96 56.17) (end 176.36 56.17) (width 1) (layer "B.Cu") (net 5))
 (segment (start 61.5 78.3) (end 62.8 77) (width 1) (layer "B.Cu") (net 5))
 (segment (start 148.45 62.36) (end 148.45 59.82) (width 1) (layer "B.Cu") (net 5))
 (segment (start 191.51 89.16) (end 191.64 89.29) (width 1) (layer "B.Cu") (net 5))
 (segment (start 204.53 59.38) (end 206.57 59.38) (width 1) (layer "B.Cu") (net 26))
 (segment (start 204.52 59.37) (end 204.53 59.38) (width 1) (layer "B.Cu") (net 26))
 (segment (start 195.91 59.37) (end 204.52 59.37) (width 1) (layer "B.Cu") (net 26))
 (segment (start 54.85 83.33) (end 52.84 83.33) (width 1) (layer "B.Cu") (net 12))
 (segment (start 58.99 93.54) (end 56.75 91.3) (width 1) (layer "B.Cu") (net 12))
 (segment (start 56.75 85.23) (end 54.85 83.33) (width 1) (layer "B.Cu") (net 12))
 (segment (start 56.75 91.3) (end 56.75 85.23) (width 1) (layer "B.Cu") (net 12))
 (segment (start 61.25 93.54) (end 58.99 93.54) (width 1) (layer "B.Cu") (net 12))
 (segment (start 64.02 88.69) (end 61.25 85.92) (width 1) (layer "B.Cu") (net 10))
 (segment (start 74.82 88.69) (end 64.02 88.69) (width 1) (layer "B.Cu") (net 10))
 (segment (start 61.25 88.46) (end 63.94 91.15) (width 1) (layer "B.Cu") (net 11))
 (segment (start 63.94 91.15) (end 69.27 91.15) (width 1) (layer "B.Cu") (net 11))
 (segment (start 61.48 81.07) (end 61.25 80.84) (width 1) (layer "F.Cu") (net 8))
 (segment (start 61.48 81.07) (end 61.25 80.84) (width 1) (layer "B.Cu") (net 8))
 (segment (start 74.82 81.07) (end 61.48 81.07) (width 1) (layer "B.Cu") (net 8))
 (segment (start 61.34 75.85) (end 61.25 75.76) (width 1) (layer "F.Cu") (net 7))
 (segment (start 178.35 54.16) (end 183.54 59.35) (width 1) (layer "B.Cu") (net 7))
 (segment (start 62.41 74.6) (end 134.7 74.6) (width 1) (layer "B.Cu") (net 7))
 (segment (start 61.25 75.76) (end 62.41 74.6) (width 1) (layer "B.Cu") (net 7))
 (segment (start 134.7 74.6) (end 145.91 63.39) (width 1) (layer "B.Cu") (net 7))
 (segment (start 147.82 54.16) (end 178.35 54.16) (width 1) (layer "B.Cu") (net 7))
 (segment (start 183.54 59.35) (end 188.27 59.35) (width 1) (layer "B.Cu") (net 7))
 (segment (start 145.91 62.36) (end 145.91 59.82) (width 1) (layer "B.Cu") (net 7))
 (segment (start 145.91 63.39) (end 145.91 62.36) (width 1) (layer "B.Cu") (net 7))
 (segment (start 145.91 59.82) (end 145.91 56.07) (width 1) (layer "B.Cu") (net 7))
 (segment (start 145.91 56.07) (end 147.82 54.16) (width 1) (layer "B.Cu") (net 7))
 (segment (start 188.27 59.35) (end 188.29 59.37) (width 1) (layer "B.Cu") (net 7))
 (segment (start 74.84 95.21) (end 74.89 95.16) (width 1) (layer "F.Cu") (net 1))
 (segment (start 61.25 91) (end 65.41 95.16) (width 1) (layer "B.Cu") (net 1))
 (segment (start 65.41 95.16) (end 74.89 95.16) (width 1) (layer "B.Cu") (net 1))
 (segment (start 61.25 83.38) (end 61.27 83.36) (width 1) (layer "F.Cu") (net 9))
 (segment (start 62.78 84.91) (end 61.25 83.38) (width 1) (layer "B.Cu") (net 9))
 (segment (start 74.85 84.91) (end 62.78 84.91) (width 1) (layer "B.Cu") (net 9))
 (segment (start 168.77 59.82) (end 168.77 62.36) (width 1) (layer "B.Cu") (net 6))
 (segment (start 182.022944 96.872944) (end 182.022944 104.327056) (width 1) (layer "B.Cu") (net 6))
 (segment (start 182.022944 104.327056) (end 179.26 107.09) (width 1) (layer "B.Cu") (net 6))
 (segment (start 168.77 62.36) (end 168.77 83.62) (width 1) (layer "B.Cu") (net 6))
 (segment (start 168.77 83.62) (end 182.022944 96.872944) (width 1) (layer "B.Cu") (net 6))
 (segment (start 164.61 106.94) (end 164.76 107.09) (width 1) (layer "B.Cu") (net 3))
 (segment (start 162.3 106.94) (end 164.61 106.94) (width 1) (layer "B.Cu") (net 3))
 (segment (start 166.23 62.36) (end 166.23 77.48) (width 1) (layer "B.Cu") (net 3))
 (segment (start 159.55 84.16) (end 159.55 104.19) (width 1) (layer "B.Cu") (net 3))
 (segment (start 159.55 104.19) (end 162.3 106.94) (width 1) (layer "B.Cu") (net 3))
 (segment (start 166.23 59.82) (end 166.23 62.36) (width 1) (layer "B.Cu") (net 3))
 (segment (start 166.23 77.48) (end 159.55 84.16) (width 1) (layer "B.Cu") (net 3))
 (segment (start 50.45 75.54) (end 53.91 72.08) (width 1) (layer "B.Cu") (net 19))
 (segment (start 47.84 85.83) (end 46.51 85.83) (width 1) (layer "B.Cu") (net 19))
 (segment (start 46.17 75.54) (end 50.45 75.54) (width 1) (layer "B.Cu") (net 19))
 (segment (start 133.65 72.08) (end 143.37 62.36) (width 1) (layer "B.Cu") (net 19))
 (segment (start 43.99 83.31) (end 43.99 77.72) (width 1) (layer "B.Cu") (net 19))
 (segment (start 46.51 85.83) (end 43.99 83.31) (width 1) (layer "B.Cu") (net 19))
 (segment (start 53.91 72.08) (end 133.65 72.08) (width 1) (layer "B.Cu") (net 19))
 (segment (start 43.99 77.72) (end 46.17 75.54) (width 1) (layer "B.Cu") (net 19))
 (segment (start 143.37 62.36) (end 143.37 59.82) (width 1) (layer "B.Cu") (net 19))
 (segment (start 154.61 83.12) (end 163.69 74.04) (width 1) (layer "B.Cu") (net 4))
 (segment (start 158.5 111.94) (end 154.61 108.05) (width 1) (layer "B.Cu") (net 4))
 (segment (start 163.69 74.04) (end 163.69 62.36) (width 1) (layer "B.Cu") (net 4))
 (segment (start 164.61 111.94) (end 158.5 111.94) (width 1) (layer "B.Cu") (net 4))
 (segment (start 164.76 112.09) (end 164.61 111.94) (width 1) (layer "B.Cu") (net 4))
 (segment (start 154.61 108.05) (end 154.61 83.12) (width 1) (layer "B.Cu") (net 4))
 (segment (start 163.69 59.82) (end 163.69 62.36) (width 1) (layer "B.Cu") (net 4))
 (segment (start 82.44 81.07) (end 82.48 81.11) (width 1) (layer "F.Cu") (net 20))
 (segment (start 150.99 62.36) (end 150.99 65.64) (width 1) (layer "B.Cu") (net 20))
 (segment (start 135.56 81.07) (end 82.44 81.07) (width 1) (layer "B.Cu") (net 20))
 (segment (start 150.99 59.82) (end 150.99 62.36) (width 1) (layer "B.Cu") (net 20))
 (segment (start 150.99 65.64) (end 135.56 81.07) (width 1) (layer "B.Cu") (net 20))
 (segment (start 178.92 89.29) (end 187.14 89.29) (width 1) (layer "B.Cu") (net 24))
 (segment (start 171.31 81.68) (end 178.92 89.29) (width 1) (layer "B.Cu") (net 24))
 (segment (start 171.31 62.36) (end 171.31 81.68) (width 1) (layer "B.Cu") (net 24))
 (segment (start 171.31 59.82) (end 171.31 62.36) (width 1) (layer "B.Cu") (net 24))
 (segment (start 133.84 95.16) (end 158.61 70.39) (width 1) (layer "B.Cu") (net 2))
 (segment (start 158.61 70.39) (end 158.61 62.36) (width 1) (layer "B.Cu") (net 2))
 (segment (start 82.51 95.16) (end 133.84 95.16) (width 1) (layer "B.Cu") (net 2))
 (segment (start 158.61 59.82) (end 158.61 62.36) (width 1) (layer "B.Cu") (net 2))
 (segment (start 180.66 73.9) (end 187.01 73.9) (width 1) (layer "B.Cu") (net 25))
 (segment (start 173.85 67.09) (end 180.66 73.9) (width 1) (layer "B.Cu") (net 25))
 (segment (start 173.85 62.36) (end 173.85 67.09) (width 1) (layer "B.Cu") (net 25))
 (segment (start 173.85 59.82) (end 173.85 62.36) (width 1) (layer "B.Cu") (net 25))
 (segment (start 135.47 88.69) (end 82.44 88.69) (width 1) (layer "B.Cu") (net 22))
 (segment (start 156.07 62.36) (end 156.07 68.09) (width 1) (layer "B.Cu") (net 22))
 (segment (start 156.07 59.82) (end 156.07 62.36) (width 1) (layer "B.Cu") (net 22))
 (segment (start 156.07 68.09) (end 135.47 88.69) (width 1) (layer "B.Cu") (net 22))
 (segment (start 161.15 59.82) (end 161.15 62.36) (width 1) (layer "B.Cu") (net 23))
 (segment (start 134.61 98.77) (end 69.27 98.77) (width 1) (layer "B.Cu") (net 23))
 (segment (start 161.15 72.23) (end 134.61 98.77) (width 1) (layer "B.Cu") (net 23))
 (segment (start 161.15 62.36) (end 161.15 72.23) (width 1) (layer "B.Cu") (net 23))
 (segment (start 82.47 84.91) (end 135.49 84.91) (width 1) (layer "B.Cu") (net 21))
 (segment (start 153.53 59.82) (end 153.53 62.36) (width 1) (layer "B.Cu") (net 21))
 (segment (start 135.49 84.91) (end 153.53 66.87) (width 1) (layer "B.Cu") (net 21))
 (segment (start 153.53 66.87) (end 153.53 62.36) (width 1) (layer "B.Cu") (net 21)))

